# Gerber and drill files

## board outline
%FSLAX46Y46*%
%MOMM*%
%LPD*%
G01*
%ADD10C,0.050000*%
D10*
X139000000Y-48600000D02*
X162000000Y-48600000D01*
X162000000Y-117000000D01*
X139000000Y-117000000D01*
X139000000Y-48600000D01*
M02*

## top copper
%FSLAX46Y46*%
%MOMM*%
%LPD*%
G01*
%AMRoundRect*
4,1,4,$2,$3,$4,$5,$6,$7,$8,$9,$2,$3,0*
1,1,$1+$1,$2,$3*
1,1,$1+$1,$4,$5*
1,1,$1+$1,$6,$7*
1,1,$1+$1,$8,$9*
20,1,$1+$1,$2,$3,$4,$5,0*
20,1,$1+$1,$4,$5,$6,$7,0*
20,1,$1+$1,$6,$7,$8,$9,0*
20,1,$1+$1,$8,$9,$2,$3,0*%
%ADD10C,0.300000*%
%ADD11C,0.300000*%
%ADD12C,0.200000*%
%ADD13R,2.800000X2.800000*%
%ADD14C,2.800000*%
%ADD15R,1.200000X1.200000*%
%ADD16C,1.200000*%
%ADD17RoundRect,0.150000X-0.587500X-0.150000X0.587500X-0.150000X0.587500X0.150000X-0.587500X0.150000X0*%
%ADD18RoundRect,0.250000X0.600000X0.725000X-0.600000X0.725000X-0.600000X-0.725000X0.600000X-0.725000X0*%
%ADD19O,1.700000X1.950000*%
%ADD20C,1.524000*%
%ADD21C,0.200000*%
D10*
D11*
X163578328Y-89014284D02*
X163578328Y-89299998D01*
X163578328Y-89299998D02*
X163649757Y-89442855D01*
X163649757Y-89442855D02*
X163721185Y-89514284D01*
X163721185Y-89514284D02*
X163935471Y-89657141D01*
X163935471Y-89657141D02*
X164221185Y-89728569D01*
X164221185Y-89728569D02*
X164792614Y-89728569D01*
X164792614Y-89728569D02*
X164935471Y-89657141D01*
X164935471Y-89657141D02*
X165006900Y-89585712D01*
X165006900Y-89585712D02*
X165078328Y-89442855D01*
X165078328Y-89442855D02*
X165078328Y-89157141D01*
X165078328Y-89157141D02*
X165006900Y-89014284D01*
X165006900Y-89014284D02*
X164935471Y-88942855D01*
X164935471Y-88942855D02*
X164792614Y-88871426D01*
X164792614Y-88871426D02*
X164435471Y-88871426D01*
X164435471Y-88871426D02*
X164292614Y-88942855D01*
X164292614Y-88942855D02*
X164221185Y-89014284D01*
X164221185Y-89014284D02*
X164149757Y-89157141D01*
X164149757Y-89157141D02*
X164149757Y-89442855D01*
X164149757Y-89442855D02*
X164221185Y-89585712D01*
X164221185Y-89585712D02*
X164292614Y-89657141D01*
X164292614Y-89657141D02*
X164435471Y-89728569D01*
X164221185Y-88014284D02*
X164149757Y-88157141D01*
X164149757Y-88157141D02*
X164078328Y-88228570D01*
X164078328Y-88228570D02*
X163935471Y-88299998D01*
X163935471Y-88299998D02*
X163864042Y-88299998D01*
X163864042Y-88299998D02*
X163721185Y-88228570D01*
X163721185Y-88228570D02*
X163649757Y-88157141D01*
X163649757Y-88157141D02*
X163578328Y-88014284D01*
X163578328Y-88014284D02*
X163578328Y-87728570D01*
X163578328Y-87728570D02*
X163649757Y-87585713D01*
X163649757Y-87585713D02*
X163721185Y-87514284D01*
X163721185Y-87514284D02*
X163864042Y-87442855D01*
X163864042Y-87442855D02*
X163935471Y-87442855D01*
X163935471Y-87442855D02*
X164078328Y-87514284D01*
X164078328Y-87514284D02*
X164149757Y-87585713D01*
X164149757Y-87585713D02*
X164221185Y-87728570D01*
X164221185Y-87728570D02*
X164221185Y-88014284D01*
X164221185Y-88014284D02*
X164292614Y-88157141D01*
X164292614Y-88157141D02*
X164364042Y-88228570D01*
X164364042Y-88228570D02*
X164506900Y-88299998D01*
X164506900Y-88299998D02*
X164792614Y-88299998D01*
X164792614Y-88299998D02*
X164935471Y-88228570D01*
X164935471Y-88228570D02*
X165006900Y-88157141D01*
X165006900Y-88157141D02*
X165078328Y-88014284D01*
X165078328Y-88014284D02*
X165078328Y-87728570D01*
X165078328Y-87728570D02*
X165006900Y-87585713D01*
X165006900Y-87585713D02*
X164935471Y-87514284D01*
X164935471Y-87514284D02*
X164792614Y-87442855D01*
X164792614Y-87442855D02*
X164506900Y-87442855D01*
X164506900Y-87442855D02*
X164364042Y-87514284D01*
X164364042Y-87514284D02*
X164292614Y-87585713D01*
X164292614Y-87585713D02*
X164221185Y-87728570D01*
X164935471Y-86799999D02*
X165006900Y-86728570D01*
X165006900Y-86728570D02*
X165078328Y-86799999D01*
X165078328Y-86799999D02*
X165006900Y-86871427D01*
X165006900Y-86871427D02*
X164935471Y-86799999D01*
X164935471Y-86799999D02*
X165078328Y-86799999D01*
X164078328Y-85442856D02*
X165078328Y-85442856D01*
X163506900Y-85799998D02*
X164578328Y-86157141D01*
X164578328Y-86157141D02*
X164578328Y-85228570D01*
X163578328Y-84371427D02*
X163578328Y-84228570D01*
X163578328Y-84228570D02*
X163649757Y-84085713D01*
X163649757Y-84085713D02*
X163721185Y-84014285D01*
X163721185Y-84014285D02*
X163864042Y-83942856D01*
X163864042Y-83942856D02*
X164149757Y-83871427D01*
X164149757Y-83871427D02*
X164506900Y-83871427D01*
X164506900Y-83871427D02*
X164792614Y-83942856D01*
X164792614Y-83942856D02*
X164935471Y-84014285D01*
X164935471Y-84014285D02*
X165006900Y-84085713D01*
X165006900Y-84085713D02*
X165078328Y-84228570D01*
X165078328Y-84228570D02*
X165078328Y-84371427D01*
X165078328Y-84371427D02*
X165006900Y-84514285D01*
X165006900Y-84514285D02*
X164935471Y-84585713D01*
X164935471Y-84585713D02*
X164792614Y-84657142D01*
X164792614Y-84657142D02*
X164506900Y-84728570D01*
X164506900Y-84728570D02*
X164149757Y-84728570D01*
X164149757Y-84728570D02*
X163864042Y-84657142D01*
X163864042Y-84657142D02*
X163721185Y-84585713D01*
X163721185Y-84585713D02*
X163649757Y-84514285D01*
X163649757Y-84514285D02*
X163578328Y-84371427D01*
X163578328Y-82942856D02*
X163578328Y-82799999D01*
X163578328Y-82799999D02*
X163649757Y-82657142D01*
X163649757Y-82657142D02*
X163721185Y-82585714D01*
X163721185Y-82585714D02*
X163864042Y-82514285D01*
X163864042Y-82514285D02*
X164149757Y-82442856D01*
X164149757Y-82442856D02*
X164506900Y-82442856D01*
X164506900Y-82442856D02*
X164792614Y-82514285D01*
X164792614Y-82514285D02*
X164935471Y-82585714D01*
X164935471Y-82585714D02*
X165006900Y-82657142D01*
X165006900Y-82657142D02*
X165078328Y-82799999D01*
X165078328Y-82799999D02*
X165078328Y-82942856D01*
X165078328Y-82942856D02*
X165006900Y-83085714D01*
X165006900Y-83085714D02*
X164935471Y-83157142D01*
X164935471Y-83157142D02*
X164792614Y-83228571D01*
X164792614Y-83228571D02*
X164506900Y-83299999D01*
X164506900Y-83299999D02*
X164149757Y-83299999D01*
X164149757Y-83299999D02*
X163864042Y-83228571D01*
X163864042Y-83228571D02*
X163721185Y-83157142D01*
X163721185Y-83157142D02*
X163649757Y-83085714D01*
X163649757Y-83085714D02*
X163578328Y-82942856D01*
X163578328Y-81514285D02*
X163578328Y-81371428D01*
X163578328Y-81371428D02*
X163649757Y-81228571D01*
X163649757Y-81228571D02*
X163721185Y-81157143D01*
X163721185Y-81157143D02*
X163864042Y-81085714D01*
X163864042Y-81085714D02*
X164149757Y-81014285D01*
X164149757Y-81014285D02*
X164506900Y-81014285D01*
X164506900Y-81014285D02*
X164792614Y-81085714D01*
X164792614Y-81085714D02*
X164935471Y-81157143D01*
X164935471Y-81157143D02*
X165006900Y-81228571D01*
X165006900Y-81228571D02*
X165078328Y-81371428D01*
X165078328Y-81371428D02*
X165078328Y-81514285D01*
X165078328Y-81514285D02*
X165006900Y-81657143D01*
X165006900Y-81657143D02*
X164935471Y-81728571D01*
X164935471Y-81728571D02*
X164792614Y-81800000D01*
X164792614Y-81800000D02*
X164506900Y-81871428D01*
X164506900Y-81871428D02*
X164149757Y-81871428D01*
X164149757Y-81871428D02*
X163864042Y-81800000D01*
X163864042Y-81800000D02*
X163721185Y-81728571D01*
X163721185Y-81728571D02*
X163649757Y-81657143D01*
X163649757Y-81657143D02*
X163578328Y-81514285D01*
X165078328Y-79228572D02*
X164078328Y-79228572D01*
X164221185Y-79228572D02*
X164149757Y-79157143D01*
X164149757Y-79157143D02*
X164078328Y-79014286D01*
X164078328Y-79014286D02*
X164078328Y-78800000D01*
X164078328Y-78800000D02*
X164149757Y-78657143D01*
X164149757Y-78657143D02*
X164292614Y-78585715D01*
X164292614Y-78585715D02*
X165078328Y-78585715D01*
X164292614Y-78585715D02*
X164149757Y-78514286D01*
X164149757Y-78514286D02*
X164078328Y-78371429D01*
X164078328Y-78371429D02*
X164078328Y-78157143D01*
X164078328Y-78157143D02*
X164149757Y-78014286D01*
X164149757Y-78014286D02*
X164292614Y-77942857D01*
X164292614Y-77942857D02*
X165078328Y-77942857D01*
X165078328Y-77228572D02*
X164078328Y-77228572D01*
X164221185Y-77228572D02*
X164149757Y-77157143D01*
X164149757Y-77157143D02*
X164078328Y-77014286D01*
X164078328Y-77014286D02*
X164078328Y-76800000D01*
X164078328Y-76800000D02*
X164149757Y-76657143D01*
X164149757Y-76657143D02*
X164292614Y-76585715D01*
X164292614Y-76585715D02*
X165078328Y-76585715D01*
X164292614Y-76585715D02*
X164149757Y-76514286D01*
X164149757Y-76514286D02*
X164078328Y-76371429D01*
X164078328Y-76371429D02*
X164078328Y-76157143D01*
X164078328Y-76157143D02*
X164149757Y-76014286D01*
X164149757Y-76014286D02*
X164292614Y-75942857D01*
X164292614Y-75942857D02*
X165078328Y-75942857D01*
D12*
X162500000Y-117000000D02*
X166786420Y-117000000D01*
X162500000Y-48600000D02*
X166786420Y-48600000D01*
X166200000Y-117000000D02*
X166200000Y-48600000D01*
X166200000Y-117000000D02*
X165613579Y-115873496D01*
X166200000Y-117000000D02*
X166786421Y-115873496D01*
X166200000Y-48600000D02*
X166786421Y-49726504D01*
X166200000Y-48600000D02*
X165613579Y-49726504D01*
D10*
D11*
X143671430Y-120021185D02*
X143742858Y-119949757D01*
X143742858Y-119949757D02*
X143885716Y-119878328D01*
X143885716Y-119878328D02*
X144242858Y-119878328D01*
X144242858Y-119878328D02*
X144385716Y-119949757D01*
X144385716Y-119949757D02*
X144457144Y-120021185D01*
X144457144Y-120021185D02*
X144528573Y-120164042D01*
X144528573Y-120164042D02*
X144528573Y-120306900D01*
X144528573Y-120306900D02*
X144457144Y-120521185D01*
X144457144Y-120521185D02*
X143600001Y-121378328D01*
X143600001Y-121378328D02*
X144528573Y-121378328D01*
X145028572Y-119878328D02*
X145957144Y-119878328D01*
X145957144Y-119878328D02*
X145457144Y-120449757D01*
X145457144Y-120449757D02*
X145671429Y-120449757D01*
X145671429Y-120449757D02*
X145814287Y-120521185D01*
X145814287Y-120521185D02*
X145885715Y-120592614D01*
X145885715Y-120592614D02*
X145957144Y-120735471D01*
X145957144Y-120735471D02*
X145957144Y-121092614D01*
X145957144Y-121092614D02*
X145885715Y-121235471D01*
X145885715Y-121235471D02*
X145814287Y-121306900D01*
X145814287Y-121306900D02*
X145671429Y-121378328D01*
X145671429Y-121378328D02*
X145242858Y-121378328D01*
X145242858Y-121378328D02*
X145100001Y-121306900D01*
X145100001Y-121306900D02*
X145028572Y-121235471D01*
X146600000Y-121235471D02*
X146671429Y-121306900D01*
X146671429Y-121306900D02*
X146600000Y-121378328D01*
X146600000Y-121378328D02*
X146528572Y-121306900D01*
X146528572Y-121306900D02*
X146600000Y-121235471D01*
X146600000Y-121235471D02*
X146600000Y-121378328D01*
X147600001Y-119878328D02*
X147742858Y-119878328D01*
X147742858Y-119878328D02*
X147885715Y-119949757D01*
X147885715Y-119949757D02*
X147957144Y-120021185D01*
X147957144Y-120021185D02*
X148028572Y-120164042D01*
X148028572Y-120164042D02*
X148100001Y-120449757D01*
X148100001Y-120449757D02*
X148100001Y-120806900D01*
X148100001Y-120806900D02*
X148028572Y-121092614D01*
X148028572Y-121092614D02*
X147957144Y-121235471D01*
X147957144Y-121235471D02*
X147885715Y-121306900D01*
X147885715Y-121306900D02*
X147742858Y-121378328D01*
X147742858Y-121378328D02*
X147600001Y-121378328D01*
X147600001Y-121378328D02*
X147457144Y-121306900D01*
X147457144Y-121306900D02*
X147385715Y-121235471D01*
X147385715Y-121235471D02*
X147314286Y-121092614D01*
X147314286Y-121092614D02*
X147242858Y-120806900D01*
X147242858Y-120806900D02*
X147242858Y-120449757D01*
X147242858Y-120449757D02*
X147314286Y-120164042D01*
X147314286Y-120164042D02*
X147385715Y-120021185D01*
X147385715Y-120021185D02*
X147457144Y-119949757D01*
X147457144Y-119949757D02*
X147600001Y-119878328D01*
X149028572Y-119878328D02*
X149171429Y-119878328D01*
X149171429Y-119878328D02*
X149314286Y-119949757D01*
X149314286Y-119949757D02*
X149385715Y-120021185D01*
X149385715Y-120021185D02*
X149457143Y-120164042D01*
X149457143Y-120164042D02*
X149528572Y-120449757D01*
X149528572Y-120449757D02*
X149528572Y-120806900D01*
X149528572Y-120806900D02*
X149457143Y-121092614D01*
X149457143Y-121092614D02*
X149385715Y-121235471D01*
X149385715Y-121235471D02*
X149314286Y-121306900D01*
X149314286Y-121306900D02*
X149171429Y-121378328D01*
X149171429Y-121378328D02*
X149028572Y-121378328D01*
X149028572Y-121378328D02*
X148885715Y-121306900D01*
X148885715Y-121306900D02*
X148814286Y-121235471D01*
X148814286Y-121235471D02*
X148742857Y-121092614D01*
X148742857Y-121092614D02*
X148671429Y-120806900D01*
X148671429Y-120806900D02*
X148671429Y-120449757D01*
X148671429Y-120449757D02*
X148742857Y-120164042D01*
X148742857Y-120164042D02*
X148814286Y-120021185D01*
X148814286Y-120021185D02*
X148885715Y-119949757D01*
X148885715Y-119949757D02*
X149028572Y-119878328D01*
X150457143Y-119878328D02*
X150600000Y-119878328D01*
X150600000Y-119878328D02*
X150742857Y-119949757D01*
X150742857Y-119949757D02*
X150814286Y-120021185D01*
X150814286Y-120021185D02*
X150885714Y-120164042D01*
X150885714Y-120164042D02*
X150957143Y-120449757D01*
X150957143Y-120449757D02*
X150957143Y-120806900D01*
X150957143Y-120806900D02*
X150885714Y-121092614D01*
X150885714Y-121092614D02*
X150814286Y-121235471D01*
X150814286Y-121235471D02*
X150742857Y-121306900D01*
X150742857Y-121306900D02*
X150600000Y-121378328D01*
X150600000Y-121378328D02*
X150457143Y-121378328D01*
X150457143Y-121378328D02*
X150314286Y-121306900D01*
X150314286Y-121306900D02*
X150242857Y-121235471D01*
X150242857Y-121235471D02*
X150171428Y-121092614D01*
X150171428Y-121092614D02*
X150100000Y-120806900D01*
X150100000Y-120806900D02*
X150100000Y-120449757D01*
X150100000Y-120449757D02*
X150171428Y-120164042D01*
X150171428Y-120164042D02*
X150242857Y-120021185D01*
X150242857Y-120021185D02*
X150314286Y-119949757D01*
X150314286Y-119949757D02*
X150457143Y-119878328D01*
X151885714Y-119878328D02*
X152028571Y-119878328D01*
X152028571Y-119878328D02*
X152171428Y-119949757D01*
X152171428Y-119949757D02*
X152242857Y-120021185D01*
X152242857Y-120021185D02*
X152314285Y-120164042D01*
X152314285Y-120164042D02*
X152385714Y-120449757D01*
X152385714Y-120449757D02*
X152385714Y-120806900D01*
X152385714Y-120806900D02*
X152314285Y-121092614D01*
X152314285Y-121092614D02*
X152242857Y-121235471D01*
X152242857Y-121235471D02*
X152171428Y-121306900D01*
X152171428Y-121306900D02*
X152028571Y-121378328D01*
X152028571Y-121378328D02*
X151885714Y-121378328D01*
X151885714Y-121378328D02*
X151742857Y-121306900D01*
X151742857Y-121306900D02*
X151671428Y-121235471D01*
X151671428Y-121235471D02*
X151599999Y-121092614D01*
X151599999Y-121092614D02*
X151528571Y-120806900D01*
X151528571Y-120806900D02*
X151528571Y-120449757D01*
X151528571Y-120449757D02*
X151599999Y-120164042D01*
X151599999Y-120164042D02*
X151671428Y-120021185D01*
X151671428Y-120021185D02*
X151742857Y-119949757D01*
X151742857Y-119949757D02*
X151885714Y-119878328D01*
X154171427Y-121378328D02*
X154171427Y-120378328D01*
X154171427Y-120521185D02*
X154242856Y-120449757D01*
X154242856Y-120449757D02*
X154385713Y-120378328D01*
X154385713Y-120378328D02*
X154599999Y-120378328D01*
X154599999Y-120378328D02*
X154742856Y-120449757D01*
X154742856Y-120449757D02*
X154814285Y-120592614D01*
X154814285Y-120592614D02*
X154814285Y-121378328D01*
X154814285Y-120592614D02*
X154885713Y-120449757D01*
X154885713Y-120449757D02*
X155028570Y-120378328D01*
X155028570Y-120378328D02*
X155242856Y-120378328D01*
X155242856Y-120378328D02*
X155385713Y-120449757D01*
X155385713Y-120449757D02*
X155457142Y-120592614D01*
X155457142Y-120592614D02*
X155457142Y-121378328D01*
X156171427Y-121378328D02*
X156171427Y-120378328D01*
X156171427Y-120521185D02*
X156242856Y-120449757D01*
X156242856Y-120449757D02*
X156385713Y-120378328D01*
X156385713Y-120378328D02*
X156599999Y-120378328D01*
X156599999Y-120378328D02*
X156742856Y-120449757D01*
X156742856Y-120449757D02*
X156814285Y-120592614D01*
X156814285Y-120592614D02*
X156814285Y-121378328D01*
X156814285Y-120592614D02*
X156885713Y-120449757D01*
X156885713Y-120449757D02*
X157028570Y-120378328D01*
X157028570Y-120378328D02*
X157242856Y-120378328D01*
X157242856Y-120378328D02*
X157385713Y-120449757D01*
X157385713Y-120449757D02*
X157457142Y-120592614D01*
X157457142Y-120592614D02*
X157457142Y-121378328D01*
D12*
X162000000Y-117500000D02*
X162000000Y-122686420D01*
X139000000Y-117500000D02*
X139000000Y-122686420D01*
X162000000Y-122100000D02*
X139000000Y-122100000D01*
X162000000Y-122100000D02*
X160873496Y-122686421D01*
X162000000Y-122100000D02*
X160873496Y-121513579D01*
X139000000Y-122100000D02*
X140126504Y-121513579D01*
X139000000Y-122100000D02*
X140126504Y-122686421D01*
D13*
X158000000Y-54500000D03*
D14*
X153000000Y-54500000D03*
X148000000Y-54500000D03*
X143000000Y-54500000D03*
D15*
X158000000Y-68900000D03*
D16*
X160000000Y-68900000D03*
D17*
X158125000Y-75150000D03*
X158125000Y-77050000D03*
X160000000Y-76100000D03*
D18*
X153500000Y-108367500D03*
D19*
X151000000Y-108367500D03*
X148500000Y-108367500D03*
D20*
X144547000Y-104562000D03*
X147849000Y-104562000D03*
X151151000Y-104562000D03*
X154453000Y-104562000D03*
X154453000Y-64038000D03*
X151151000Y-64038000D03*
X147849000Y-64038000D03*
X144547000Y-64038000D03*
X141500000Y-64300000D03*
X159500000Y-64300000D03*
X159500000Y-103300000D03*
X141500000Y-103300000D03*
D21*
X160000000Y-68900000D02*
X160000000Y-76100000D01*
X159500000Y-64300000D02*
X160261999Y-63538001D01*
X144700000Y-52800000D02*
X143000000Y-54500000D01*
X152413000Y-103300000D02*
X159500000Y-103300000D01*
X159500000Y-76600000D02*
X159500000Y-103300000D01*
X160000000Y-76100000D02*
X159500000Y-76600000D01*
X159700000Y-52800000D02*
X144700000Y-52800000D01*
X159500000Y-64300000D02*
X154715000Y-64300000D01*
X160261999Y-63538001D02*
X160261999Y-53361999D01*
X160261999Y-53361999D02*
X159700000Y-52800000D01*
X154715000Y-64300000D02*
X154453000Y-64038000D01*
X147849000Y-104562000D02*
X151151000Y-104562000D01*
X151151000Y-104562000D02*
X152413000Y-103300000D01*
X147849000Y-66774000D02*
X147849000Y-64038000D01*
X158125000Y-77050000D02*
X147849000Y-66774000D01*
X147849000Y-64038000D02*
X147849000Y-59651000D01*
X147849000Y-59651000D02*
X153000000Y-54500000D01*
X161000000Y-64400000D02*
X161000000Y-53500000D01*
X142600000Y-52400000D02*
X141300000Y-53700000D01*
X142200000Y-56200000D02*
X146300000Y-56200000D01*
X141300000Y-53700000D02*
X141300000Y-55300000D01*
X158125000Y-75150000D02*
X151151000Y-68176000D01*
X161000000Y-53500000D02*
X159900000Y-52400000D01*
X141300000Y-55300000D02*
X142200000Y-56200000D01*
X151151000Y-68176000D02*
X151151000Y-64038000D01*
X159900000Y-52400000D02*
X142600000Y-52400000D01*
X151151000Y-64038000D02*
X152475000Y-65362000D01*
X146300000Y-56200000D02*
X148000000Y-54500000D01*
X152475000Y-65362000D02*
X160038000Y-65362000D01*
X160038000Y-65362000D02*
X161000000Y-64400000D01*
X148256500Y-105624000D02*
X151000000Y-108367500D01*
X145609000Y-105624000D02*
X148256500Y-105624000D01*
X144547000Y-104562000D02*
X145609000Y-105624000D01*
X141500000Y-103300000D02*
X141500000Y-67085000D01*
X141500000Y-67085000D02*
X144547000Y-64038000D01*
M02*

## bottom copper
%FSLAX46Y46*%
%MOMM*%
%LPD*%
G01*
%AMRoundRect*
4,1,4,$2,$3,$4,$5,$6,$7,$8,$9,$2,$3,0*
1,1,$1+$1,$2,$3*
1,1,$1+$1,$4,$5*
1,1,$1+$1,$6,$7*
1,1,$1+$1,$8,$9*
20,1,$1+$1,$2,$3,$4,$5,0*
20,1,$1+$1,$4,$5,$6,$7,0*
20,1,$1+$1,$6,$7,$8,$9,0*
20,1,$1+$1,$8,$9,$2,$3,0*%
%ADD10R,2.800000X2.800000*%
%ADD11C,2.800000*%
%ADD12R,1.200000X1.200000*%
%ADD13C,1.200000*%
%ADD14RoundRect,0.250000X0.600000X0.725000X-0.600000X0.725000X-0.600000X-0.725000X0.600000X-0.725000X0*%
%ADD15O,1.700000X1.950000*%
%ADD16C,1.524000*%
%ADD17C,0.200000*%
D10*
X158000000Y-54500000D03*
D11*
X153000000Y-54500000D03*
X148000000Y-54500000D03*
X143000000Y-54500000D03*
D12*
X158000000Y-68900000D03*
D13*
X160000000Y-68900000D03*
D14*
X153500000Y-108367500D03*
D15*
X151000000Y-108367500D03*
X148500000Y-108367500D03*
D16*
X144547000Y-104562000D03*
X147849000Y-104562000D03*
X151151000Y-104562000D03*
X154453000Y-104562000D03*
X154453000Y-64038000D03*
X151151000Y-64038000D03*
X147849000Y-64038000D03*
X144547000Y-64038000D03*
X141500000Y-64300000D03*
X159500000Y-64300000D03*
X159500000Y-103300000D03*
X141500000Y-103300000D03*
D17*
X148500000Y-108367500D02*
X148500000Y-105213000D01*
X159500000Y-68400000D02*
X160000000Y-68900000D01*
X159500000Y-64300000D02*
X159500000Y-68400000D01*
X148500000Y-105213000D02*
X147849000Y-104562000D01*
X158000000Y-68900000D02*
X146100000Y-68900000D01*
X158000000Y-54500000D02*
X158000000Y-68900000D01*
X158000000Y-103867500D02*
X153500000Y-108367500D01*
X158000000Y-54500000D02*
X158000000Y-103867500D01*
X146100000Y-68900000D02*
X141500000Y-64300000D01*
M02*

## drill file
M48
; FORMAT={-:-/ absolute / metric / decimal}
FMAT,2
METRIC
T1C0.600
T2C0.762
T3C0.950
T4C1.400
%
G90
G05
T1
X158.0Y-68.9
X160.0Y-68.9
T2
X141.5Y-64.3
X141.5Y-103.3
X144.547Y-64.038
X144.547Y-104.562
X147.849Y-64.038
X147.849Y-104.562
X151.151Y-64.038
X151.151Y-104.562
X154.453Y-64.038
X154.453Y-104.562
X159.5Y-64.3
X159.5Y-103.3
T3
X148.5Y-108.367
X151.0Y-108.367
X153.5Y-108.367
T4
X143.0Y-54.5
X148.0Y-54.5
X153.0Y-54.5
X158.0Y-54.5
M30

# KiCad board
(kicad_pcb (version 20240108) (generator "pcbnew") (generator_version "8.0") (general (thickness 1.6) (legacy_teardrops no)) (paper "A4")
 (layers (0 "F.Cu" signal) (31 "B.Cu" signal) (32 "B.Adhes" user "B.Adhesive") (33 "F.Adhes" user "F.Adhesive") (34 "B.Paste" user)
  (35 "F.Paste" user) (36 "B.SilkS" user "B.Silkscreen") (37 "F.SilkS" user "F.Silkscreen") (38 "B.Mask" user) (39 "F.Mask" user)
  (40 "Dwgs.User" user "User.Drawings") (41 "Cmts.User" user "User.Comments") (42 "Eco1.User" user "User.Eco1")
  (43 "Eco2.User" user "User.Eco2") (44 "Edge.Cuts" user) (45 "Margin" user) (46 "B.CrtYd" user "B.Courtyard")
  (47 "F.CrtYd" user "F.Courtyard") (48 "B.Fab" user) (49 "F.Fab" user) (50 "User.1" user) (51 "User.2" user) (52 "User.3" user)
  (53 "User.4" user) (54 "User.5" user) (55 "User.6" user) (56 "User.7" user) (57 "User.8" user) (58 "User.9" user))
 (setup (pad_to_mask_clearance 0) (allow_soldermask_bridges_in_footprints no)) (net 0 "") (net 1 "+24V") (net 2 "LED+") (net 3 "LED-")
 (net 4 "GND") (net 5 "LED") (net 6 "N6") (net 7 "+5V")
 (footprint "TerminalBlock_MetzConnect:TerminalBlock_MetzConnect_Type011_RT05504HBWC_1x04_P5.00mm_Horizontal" (layer "F.Cu")
  (at 158 54.5 180)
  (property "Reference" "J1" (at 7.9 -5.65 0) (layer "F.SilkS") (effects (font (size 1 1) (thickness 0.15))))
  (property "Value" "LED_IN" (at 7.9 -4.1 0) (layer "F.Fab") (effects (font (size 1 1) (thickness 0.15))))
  (pad "1" thru_hole rect (at 0 0 180) (size 2.8 2.8) (drill 1.4) (layers "*.Cu" "*.Mask") (remove_unused_layers no) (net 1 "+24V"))
  (pad "2" thru_hole circle (at 5 0 180) (size 2.8 2.8) (drill 1.4) (layers "*.Cu" "*.Mask") (remove_unused_layers no) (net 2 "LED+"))
  (pad "3" thru_hole circle (at 10 0 180) (size 2.8 2.8) (drill 1.4) (layers "*.Cu" "*.Mask") (remove_unused_layers no) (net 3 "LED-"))
  (pad "4" thru_hole circle (at 15 0 180) (size 2.8 2.8) (drill 1.4) (layers "*.Cu" "*.Mask") (remove_unused_layers no) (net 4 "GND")))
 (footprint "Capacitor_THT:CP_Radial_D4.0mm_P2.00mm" (layer "F.Cu") (at 158 68.9)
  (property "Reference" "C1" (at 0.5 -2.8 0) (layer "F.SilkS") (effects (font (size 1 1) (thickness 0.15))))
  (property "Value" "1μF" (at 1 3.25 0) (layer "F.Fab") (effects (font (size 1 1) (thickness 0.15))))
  (pad "1" thru_hole rect (at 0 0) (size 1.2 1.2) (drill 0.6) (layers "*.Cu" "*.Mask") (remove_unused_layers no) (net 1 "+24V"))
  (pad "2" thru_hole circle (at 2 0) (size 1.2 1.2) (drill 0.6) (layers "*.Cu" "*.Mask") (remove_unused_layers no) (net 4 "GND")))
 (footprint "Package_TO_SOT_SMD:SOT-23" (layer "F.Cu") (at 159.0625 76.1)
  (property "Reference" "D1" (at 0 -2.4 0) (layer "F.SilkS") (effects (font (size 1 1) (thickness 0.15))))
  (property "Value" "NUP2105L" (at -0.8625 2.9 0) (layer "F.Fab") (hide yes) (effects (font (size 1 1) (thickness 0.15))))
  (pad "1" smd roundrect (at -0.9375 -0.95) (size 1.475 0.6) (layers "F.Cu" "F.Paste" "F.Mask") (roundrect_rratio 0.25) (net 3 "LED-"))
  (pad "2" smd roundrect (at -0.9375 0.95) (size 1.475 0.6) (layers "F.Cu" "F.Paste" "F.Mask") (roundrect_rratio 0.25) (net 2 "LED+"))
  (pad "3" smd roundrect (at 0.9375 0) (size 1.475 0.6) (layers "F.Cu" "F.Paste" "F.Mask") (roundrect_rratio 0.25) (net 4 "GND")))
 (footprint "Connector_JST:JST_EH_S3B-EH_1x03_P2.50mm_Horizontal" (layer "F.Cu") (at 153.5 108.3675 180)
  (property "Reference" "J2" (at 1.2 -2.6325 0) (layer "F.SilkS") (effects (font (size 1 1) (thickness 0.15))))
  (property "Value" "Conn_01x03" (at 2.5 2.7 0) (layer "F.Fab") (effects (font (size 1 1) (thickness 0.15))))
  (pad "1" thru_hole roundrect (at 0 0 180) (size 1.7 1.95) (drill 0.95) (layers "*.Cu" "*.Mask") (remove_unused_layers no)
   (roundrect_rratio 0.147059) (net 1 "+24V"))
  (pad "2" thru_hole oval (at 2.5 0 180) (size 1.7 1.95) (drill 0.95) (layers "*.Cu" "*.Mask") (remove_unused_layers no) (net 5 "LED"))
  (pad "3" thru_hole oval (at 5 0 180) (size 1.7 1.95) (drill 0.95) (layers "*.Cu" "*.Mask") (remove_unused_layers no) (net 4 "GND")))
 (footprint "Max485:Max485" (layer "F.Cu") (at 149 84.2 -90)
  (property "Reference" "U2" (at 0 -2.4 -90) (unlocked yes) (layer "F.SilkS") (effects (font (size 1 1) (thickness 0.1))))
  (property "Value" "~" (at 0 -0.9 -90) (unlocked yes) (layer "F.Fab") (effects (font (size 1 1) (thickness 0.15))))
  (pad "1" thru_hole circle (at 20.362 4.453) (size 1.524 1.524) (drill 0.762) (layers "*.Cu" "*.Mask") (remove_unused_layers no)
   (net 5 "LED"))
  (pad "2" thru_hole circle (at 20.362 1.151) (size 1.524 1.524) (drill 0.762) (layers "*.Cu" "*.Mask") (remove_unused_layers no)
   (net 4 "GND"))
  (pad "3" thru_hole circle (at 20.362 -2.151) (size 1.524 1.524) (drill 0.762) (layers "*.Cu" "*.Mask") (remove_unused_layers no)
   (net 4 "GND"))
  (pad "4" thru_hole circle (at 20.362 -5.453) (size 1.524 1.524) (drill 0.762) (layers "*.Cu" "*.Mask") (remove_unused_layers no)
   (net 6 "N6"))
  (pad "5" thru_hole circle (at -20.162 -5.453) (size 1.524 1.524) (drill 0.762) (layers "*.Cu" "*.Mask") (remove_unused_layers no)
   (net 4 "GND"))
  (pad "6" thru_hole circle (at -20.162 -2.151) (size 1.524 1.524) (drill 0.762) (layers "*.Cu" "*.Mask") (remove_unused_layers no)
   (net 3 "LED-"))
  (pad "7" thru_hole circle (at -20.162 1.151) (size 1.524 1.524) (drill 0.762) (layers "*.Cu" "*.Mask") (remove_unused_layers no)
   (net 2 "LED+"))
  (pad "8" thru_hole circle (at -20.162 4.453) (size 1.524 1.524) (drill 0.762) (layers "*.Cu" "*.Mask") (remove_unused_layers no)
   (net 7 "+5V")))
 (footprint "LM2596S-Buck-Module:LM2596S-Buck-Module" (layer "B.Cu") (at 150.5 83.8 -90)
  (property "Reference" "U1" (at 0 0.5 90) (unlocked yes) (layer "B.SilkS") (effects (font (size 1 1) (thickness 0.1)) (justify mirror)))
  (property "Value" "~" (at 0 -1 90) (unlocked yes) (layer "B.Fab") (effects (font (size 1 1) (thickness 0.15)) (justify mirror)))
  (pad "1" thru_hole circle (at -19.5 9 270) (size 1.524 1.524) (drill 0.762) (layers "*.Cu" "*.Mask") (remove_unused_layers no)
   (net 1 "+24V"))
  (pad "2" thru_hole circle (at -19.5 -9 270) (size 1.524 1.524) (drill 0.762) (layers "*.Cu" "*.Mask") (remove_unused_layers no)
   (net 4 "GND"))
  (pad "3" thru_hole circle (at 19.5 -9 270) (size 1.524 1.524) (drill 0.762) (layers "*.Cu" "*.Mask") (remove_unused_layers no)
   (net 4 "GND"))
  (pad "4" thru_hole circle (at 19.5 9 270) (size 1.524 1.524) (drill 0.762) (layers "*.Cu" "*.Mask") (remove_unused_layers no)
   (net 7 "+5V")))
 (gr_rect (start 139 48.6) (end 162 117) (stroke (width 0.05) (type default)) (fill none) (layer "Edge.Cuts"))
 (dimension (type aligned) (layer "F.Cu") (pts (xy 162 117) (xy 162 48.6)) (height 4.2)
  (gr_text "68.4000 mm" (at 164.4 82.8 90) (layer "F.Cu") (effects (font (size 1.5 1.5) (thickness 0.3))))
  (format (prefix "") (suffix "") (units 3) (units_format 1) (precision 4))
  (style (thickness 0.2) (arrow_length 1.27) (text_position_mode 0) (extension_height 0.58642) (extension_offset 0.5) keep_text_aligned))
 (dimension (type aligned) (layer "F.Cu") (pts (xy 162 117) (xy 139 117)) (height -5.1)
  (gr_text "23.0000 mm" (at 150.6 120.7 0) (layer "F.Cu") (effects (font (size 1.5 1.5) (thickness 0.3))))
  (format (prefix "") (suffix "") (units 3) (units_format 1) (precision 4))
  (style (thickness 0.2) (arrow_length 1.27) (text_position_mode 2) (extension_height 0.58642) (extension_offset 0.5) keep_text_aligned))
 (segment (start 160 68.9) (end 160 76.1) (width 0.2) (layer "F.Cu") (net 4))
 (segment (start 159.5 64.3) (end 160.261999 63.538001) (width 0.2) (layer "F.Cu") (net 4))
 (segment (start 144.7 52.8) (end 143 54.5) (width 0.2) (layer "F.Cu") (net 4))
 (segment (start 152.413 103.3) (end 159.5 103.3) (width 0.2) (layer "F.Cu") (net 4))
 (segment (start 159.5 76.6) (end 159.5 103.3) (width 0.2) (layer "F.Cu") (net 4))
 (segment (start 160 76.1) (end 159.5 76.6) (width 0.2) (layer "F.Cu") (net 4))
 (segment (start 159.7 52.8) (end 144.7 52.8) (width 0.2) (layer "F.Cu") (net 4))
 (segment (start 159.5 64.3) (end 154.715 64.3) (width 0.2) (layer "F.Cu") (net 4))
 (segment (start 160.261999 63.538001) (end 160.261999 53.361999) (width 0.2) (layer "F.Cu") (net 4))
 (segment (start 160.261999 53.361999) (end 159.7 52.8) (width 0.2) (layer "F.Cu") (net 4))
 (segment (start 154.715 64.3) (end 154.453 64.038) (width 0.2) (layer "F.Cu") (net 4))
 (segment (start 147.849 104.562) (end 151.151 104.562) (width 0.2) (layer "F.Cu") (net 4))
 (segment (start 151.151 104.562) (end 152.413 103.3) (width 0.2) (layer "F.Cu") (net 4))
 (segment (start 148.5 108.3675) (end 148.5 105.213) (width 0.2) (layer "B.Cu") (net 4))
 (segment (start 159.5 68.4) (end 160 68.9) (width 0.2) (layer "B.Cu") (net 4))
 (segment (start 159.5 64.3) (end 159.5 68.4) (width 0.2) (layer "B.Cu") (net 4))
 (segment (start 148.5 105.213) (end 147.849 104.562) (width 0.2) (layer "B.Cu") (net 4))
 (segment (start 158 68.9) (end 146.1 68.9) (width 0.2) (layer "B.Cu") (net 1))
 (segment (start 158 54.5) (end 158 68.9) (width 0.2) (layer "B.Cu") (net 1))
 (segment (start 158 103.8675) (end 153.5 108.3675) (width 0.2) (layer "B.Cu") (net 1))
 (segment (start 158 54.5) (end 158 103.8675) (width 0.2) (layer "B.Cu") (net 1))
 (segment (start 146.1 68.9) (end 141.5 64.3) (width 0.2) (layer "B.Cu") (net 1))
 (segment (start 147.849 66.774) (end 147.849 64.038) (width 0.2) (layer "F.Cu") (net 2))
 (segment (start 158.125 77.05) (end 147.849 66.774) (width 0.2) (layer "F.Cu") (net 2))
 (segment (start 147.849 64.038) (end 147.849 59.651) (width 0.2) (layer "F.Cu") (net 2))
 (segment (start 147.849 59.651) (end 153 54.5) (width 0.2) (layer "F.Cu") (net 2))
 (segment (start 161 64.4) (end 161 53.5) (width 0.2) (layer "F.Cu") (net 3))
 (segment (start 142.6 52.4) (end 141.3 53.7) (width 0.2) (layer "F.Cu") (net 3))
 (segment (start 142.2 56.2) (end 146.3 56.2) (width 0.2) (layer "F.Cu") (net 3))
 (segment (start 141.3 53.7) (end 141.3 55.3) (width 0.2) (layer "F.Cu") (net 3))
 (segment (start 158.125 75.15) (end 151.151 68.176) (width 0.2) (layer "F.Cu") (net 3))
 (segment (start 161 53.5) (end 159.9 52.4) (width 0.2) (layer "F.Cu") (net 3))
 (segment (start 141.3 55.3) (end 142.2 56.2) (width 0.2) (layer "F.Cu") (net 3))
 (segment (start 151.151 68.176) (end 151.151 64.038) (width 0.2) (layer "F.Cu") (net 3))
 (segment (start 159.9 52.4) (end 142.6 52.4) (width 0.2) (layer "F.Cu") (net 3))
 (segment (start 151.151 64.038) (end 152.475 65.362) (width 0.2) (layer "F.Cu") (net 3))
 (segment (start 146.3 56.2) (end 148 54.5) (width 0.2) (layer "F.Cu") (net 3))
 (segment (start 152.475 65.362) (end 160.038 65.362) (width 0.2) (layer "F.Cu") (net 3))
 (segment (start 160.038 65.362) (end 161 64.4) (width 0.2) (layer "F.Cu") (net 3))
 (segment (start 148.2565 105.624) (end 151 108.3675) (width 0.2) (layer "F.Cu") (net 5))
 (segment (start 145.609 105.624) (end 148.2565 105.624) (width 0.2) (layer "F.Cu") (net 5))
 (segment (start 144.547 104.562) (end 145.609 105.624) (width 0.2) (layer "F.Cu") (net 5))
 (segment (start 141.5 103.3) (end 141.5 67.085) (width 0.2) (layer "F.Cu") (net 7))
 (segment (start 141.5 67.085) (end 144.547 64.038) (width 0.2) (layer "F.Cu") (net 7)))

